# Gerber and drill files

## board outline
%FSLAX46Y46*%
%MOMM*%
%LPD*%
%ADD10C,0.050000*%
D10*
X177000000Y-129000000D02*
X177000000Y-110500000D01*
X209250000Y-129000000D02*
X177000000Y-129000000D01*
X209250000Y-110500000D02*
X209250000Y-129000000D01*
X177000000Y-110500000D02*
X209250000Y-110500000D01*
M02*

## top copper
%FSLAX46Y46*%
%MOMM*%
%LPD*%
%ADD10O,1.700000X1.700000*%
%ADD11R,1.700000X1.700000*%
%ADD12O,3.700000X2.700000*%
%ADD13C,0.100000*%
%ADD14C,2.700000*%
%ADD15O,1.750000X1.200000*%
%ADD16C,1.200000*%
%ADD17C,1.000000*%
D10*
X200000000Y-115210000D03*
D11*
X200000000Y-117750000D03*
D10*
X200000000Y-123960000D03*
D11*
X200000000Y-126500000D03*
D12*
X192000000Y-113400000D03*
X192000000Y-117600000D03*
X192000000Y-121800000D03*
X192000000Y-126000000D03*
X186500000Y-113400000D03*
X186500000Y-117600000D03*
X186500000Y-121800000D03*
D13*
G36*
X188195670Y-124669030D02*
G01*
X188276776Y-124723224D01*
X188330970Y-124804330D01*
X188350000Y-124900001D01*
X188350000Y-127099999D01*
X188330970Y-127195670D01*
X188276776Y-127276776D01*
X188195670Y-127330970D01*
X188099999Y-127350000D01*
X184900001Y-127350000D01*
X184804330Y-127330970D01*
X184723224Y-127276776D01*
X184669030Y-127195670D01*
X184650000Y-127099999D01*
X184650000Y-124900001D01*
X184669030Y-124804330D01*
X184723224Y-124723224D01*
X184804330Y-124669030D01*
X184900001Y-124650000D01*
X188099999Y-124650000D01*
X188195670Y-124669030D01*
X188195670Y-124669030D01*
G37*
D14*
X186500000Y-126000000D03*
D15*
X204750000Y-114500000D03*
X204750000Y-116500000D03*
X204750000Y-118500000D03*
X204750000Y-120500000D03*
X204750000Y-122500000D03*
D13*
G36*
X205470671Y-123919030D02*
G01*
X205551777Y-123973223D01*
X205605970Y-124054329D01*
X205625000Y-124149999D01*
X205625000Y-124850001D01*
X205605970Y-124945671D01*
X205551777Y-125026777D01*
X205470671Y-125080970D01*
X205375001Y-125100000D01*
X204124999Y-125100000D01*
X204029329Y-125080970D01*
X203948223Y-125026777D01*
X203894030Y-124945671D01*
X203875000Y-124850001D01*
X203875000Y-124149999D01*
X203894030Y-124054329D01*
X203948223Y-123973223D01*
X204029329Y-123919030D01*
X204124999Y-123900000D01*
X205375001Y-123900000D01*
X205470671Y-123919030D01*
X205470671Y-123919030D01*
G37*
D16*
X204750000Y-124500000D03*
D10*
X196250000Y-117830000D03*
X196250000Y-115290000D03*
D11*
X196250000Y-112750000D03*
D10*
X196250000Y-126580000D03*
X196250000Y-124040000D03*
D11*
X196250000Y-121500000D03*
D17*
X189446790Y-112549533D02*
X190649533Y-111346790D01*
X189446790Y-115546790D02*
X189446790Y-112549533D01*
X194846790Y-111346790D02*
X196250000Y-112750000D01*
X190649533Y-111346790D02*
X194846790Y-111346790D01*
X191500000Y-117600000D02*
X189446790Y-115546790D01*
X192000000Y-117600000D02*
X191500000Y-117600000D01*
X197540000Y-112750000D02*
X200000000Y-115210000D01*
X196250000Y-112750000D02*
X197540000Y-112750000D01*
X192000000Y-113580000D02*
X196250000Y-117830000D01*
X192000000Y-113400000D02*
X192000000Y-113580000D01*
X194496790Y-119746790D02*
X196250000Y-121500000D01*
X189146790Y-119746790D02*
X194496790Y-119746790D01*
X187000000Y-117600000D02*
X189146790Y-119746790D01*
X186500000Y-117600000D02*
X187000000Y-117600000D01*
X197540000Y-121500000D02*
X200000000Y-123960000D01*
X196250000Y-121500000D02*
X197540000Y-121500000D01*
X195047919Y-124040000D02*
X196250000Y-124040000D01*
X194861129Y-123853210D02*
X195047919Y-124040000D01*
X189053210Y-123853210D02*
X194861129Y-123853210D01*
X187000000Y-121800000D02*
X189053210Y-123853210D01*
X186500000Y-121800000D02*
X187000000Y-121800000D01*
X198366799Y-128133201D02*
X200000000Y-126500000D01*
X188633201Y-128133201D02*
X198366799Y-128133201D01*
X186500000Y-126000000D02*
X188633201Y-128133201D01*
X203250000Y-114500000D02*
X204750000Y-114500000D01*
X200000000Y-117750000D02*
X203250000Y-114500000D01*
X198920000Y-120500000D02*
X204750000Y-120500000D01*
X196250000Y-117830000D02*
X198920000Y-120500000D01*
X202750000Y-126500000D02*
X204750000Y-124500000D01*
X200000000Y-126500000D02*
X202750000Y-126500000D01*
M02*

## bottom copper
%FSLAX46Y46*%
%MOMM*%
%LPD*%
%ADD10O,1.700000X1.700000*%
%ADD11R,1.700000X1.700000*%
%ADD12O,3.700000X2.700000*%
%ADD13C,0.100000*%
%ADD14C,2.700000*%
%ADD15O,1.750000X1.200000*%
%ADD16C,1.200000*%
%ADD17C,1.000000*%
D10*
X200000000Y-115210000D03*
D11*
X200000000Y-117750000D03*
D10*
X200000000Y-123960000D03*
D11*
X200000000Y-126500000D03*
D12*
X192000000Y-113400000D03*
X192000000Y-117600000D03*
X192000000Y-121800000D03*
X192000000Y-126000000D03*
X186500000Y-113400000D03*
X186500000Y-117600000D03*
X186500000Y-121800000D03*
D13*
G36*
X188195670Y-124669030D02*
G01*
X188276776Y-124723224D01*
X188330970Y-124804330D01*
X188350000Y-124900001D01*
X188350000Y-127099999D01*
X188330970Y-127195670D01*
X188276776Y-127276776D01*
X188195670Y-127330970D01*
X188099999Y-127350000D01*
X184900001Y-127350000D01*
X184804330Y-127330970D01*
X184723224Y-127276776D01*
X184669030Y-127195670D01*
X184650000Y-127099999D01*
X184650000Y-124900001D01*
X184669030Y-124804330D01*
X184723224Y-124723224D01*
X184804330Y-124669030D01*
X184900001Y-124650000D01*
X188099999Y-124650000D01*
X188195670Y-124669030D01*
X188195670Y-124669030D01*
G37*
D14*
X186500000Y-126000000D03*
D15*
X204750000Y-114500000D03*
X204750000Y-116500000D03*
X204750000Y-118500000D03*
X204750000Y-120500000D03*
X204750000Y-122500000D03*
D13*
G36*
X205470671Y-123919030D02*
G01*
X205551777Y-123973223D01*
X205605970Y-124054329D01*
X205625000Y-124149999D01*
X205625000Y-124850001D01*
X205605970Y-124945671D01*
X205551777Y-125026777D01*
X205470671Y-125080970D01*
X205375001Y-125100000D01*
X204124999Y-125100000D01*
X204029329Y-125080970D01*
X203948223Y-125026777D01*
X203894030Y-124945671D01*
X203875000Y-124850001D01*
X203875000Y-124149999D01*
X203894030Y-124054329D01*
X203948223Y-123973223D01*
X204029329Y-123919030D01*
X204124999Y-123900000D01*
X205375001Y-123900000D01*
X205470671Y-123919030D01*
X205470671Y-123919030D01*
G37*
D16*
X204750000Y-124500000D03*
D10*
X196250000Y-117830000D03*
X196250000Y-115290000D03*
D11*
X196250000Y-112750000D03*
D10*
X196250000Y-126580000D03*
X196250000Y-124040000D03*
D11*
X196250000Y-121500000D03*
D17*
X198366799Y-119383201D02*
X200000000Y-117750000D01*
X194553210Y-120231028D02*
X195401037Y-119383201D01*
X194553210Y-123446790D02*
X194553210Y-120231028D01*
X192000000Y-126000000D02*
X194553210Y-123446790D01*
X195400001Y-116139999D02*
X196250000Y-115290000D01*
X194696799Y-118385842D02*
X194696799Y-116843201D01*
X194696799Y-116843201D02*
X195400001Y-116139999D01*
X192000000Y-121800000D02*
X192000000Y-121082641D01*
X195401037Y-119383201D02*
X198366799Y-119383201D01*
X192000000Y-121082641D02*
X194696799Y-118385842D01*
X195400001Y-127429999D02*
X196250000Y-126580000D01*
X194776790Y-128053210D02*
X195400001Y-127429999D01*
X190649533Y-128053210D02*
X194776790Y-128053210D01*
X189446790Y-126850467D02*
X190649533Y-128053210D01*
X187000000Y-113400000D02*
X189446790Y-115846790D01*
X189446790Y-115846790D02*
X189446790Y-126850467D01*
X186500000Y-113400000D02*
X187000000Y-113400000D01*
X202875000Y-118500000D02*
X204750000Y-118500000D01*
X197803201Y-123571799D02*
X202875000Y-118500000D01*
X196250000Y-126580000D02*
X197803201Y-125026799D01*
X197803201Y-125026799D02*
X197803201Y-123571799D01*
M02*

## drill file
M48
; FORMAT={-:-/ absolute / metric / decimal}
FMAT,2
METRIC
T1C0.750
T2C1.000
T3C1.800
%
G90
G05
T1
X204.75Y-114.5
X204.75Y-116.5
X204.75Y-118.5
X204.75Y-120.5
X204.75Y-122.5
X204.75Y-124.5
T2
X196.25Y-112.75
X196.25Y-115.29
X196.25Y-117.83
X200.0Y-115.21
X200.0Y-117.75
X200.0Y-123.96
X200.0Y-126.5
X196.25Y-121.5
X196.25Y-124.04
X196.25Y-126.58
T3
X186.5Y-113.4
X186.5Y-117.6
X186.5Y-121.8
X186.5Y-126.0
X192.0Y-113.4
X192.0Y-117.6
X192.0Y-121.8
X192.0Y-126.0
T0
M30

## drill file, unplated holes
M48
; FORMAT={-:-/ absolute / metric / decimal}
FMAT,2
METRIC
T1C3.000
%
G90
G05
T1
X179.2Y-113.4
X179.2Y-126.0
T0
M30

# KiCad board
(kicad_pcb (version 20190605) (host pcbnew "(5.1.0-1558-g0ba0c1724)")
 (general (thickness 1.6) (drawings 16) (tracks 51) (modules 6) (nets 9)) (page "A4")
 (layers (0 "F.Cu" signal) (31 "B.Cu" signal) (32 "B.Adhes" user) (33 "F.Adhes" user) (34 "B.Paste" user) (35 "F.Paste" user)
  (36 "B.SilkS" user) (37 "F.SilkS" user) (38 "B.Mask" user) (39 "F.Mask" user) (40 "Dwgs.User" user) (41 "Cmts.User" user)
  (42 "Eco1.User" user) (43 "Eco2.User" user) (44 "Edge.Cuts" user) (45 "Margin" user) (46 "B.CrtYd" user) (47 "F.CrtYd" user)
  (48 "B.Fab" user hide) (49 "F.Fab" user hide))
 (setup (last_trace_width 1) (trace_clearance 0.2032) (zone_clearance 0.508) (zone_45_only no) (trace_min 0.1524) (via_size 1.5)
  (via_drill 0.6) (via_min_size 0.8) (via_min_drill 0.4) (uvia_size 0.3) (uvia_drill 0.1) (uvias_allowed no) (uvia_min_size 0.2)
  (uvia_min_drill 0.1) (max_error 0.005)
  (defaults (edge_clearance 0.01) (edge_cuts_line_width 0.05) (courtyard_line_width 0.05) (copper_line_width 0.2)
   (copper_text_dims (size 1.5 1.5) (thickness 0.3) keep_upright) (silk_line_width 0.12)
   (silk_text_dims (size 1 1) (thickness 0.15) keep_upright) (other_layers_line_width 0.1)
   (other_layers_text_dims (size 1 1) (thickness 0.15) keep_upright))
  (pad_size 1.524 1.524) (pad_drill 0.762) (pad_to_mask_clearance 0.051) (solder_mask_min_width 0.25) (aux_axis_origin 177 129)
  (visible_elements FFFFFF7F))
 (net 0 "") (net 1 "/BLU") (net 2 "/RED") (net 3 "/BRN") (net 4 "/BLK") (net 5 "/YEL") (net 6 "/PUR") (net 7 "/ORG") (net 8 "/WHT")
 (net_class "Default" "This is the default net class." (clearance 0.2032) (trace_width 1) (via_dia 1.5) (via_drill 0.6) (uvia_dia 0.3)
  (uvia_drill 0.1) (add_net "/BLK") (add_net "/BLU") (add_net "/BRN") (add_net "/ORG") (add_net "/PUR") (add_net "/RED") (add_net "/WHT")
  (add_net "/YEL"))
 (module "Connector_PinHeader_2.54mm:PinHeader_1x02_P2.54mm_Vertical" (layer "F.Cu") (at 200 117.75 180)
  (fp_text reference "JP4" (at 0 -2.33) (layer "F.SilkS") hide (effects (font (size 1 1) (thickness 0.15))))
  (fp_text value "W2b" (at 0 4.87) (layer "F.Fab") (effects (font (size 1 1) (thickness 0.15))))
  (pad "2" thru_hole oval (at 0 2.54 180) (size 1.7 1.7) (drill 1) (layers *.Cu *.Mask) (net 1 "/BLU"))
  (pad "1" thru_hole rect (at 0 0 180) (size 1.7 1.7) (drill 1) (layers *.Cu *.Mask) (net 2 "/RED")))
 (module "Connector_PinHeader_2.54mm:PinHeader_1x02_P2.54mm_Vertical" (layer "F.Cu") (at 200 126.5 180)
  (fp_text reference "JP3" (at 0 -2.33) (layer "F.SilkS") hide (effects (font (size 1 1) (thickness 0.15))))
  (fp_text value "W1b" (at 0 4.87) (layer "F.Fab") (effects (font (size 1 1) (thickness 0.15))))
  (pad "2" thru_hole oval (at 0 2.54 180) (size 1.7 1.7) (drill 1) (layers *.Cu *.Mask) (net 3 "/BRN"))
  (pad "1" thru_hole rect (at 0 0 180) (size 1.7 1.7) (drill 1) (layers *.Cu *.Mask) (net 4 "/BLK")))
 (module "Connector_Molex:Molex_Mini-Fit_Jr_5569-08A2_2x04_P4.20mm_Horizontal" (layer "F.Cu") (at 186.5 126 90)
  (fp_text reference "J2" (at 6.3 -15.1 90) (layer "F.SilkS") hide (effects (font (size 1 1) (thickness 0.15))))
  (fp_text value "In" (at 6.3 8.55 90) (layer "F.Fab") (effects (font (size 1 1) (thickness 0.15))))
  (pad "" np_thru_hole circle (at 12.6 -7.3 90) (size 3 3) (drill 3) (layers *.Cu *.Mask))
  (pad "" np_thru_hole circle (at 0 -7.3 90) (size 3 3) (drill 3) (layers *.Cu *.Mask))
  (pad "8" thru_hole oval (at 12.6 5.5 90) (size 2.7 3.7) (drill 1.8) (layers *.Cu *.Mask) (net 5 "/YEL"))
  (pad "7" thru_hole oval (at 8.4 5.5 90) (size 2.7 3.7) (drill 1.8) (layers *.Cu *.Mask) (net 1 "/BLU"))
  (pad "6" thru_hole oval (at 4.2 5.5 90) (size 2.7 3.7) (drill 1.8) (layers *.Cu *.Mask) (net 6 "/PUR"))
  (pad "5" thru_hole oval (at 0 5.5 90) (size 2.7 3.7) (drill 1.8) (layers *.Cu *.Mask) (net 2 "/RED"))
  (pad "4" thru_hole oval (at 12.6 0 90) (size 2.7 3.7) (drill 1.8) (layers *.Cu *.Mask) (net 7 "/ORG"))
  (pad "3" thru_hole oval (at 8.4 0 90) (size 2.7 3.7) (drill 1.8) (layers *.Cu *.Mask) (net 3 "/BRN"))
  (pad "2" thru_hole oval (at 4.2 0 90) (size 2.7 3.7) (drill 1.8) (layers *.Cu *.Mask) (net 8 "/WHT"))
  (pad "1" thru_hole roundrect (at 0 0 90) (size 2.7 3.7) (drill 1.8) (layers *.Cu *.Mask) (roundrect_rratio 0.09259299999999999)
   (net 4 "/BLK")))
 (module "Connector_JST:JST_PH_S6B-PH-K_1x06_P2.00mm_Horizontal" (layer "F.Cu") (at 204.75 124.5 90)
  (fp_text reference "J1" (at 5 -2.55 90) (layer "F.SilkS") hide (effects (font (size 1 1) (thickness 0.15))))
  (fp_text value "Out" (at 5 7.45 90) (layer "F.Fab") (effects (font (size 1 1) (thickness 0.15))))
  (pad "6" thru_hole oval (at 10 0 90) (size 1.2 1.75) (drill 0.75) (layers *.Cu *.Mask) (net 2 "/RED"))
  (pad "5" thru_hole oval (at 8 0 90) (size 1.2 1.75) (drill 0.75) (layers *.Cu *.Mask))
  (pad "4" thru_hole oval (at 6 0 90) (size 1.2 1.75) (drill 0.75) (layers *.Cu *.Mask) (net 7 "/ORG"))
  (pad "3" thru_hole oval (at 4 0 90) (size 1.2 1.75) (drill 0.75) (layers *.Cu *.Mask) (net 5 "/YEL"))
  (pad "2" thru_hole oval (at 2 0 90) (size 1.2 1.75) (drill 0.75) (layers *.Cu *.Mask))
  (pad "1" thru_hole roundrect (at 0 0 90) (size 1.2 1.75) (drill 0.75) (layers *.Cu *.Mask) (roundrect_rratio 0.208333) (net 4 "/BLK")))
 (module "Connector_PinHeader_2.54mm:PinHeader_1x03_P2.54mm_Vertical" (layer "F.Cu") (at 196.25 112.75)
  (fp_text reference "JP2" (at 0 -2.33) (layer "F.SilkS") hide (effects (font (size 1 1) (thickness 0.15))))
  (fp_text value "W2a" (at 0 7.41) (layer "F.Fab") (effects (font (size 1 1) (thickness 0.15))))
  (pad "3" thru_hole oval (at 0 5.08) (size 1.7 1.7) (drill 1) (layers *.Cu *.Mask) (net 5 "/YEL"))
  (pad "2" thru_hole oval (at 0 2.54) (size 1.7 1.7) (drill 1) (layers *.Cu *.Mask) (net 6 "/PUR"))
  (pad "1" thru_hole rect (at 0 0) (size 1.7 1.7) (drill 1) (layers *.Cu *.Mask) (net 1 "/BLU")))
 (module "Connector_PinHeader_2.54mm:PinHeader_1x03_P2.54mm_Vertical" (layer "F.Cu") (at 196.25 121.5)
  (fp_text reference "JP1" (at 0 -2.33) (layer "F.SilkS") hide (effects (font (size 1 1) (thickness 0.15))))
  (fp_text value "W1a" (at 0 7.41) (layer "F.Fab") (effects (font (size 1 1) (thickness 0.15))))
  (pad "3" thru_hole oval (at 0 5.08) (size 1.7 1.7) (drill 1) (layers *.Cu *.Mask) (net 7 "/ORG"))
  (pad "2" thru_hole oval (at 0 2.54) (size 1.7 1.7) (drill 1) (layers *.Cu *.Mask) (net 8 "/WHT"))
  (pad "1" thru_hole rect (at 0 0) (size 1.7 1.7) (drill 1) (layers *.Cu *.Mask) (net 3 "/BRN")))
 (gr_line (start 177 129) (end 177 110.5) (layer "Edge.Cuts") (width 0.05))
 (gr_line (start 209.25 129) (end 177 129) (layer "Edge.Cuts") (width 0.05))
 (gr_line (start 209.25 110.5) (end 209.25 129) (layer "Edge.Cuts") (width 0.05))
 (gr_line (start 177 110.5) (end 209.25 110.5) (layer "Edge.Cuts") (width 0.05))
 (segment (start 189.44679 112.549533) (end 190.649533 111.34679) (width 1) (layer "F.Cu") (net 1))
 (segment (start 189.44679 115.54679) (end 189.44679 112.549533) (width 1) (layer "F.Cu") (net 1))
 (segment (start 194.84679 111.34679) (end 196.25 112.75) (width 1) (layer "F.Cu") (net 1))
 (segment (start 190.649533 111.34679) (end 194.84679 111.34679) (width 1) (layer "F.Cu") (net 1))
 (segment (start 191.5 117.6) (end 189.44679 115.54679) (width 1) (layer "F.Cu") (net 1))
 (segment (start 192 117.6) (end 191.5 117.6) (width 1) (layer "F.Cu") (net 1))
 (segment (start 197.54 112.75) (end 200 115.21) (width 1) (layer "F.Cu") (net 1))
 (segment (start 196.25 112.75) (end 197.54 112.75) (width 1) (layer "F.Cu") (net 1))
 (segment (start 192 113.58) (end 196.25 117.83) (width 1) (layer "F.Cu") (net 5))
 (segment (start 192 113.4) (end 192 113.58) (width 1) (layer "F.Cu") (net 5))
 (segment (start 194.49679 119.74679) (end 196.25 121.5) (width 1) (layer "F.Cu") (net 3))
 (segment (start 189.14679 119.74679) (end 194.49679 119.74679) (width 1) (layer "F.Cu") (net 3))
 (segment (start 187 117.6) (end 189.14679 119.74679) (width 1) (layer "F.Cu") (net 3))
 (segment (start 186.5 117.6) (end 187 117.6) (width 1) (layer "F.Cu") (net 3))
 (segment (start 197.54 121.5) (end 200 123.96) (width 1) (layer "F.Cu") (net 3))
 (segment (start 196.25 121.5) (end 197.54 121.5) (width 1) (layer "F.Cu") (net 3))
 (segment (start 195.047919 124.04) (end 196.25 124.04) (width 1) (layer "F.Cu") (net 8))
 (segment (start 194.861129 123.85321) (end 195.047919 124.04) (width 1) (layer "F.Cu") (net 8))
 (segment (start 189.05321 123.85321) (end 194.861129 123.85321) (width 1) (layer "F.Cu") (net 8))
 (segment (start 187 121.8) (end 189.05321 123.85321) (width 1) (layer "F.Cu") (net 8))
 (segment (start 186.5 121.8) (end 187 121.8) (width 1) (layer "F.Cu") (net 8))
 (segment (start 198.366799 128.133201) (end 200 126.5) (width 1) (layer "F.Cu") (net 4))
 (segment (start 188.633201 128.133201) (end 198.366799 128.133201) (width 1) (layer "F.Cu") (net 4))
 (segment (start 186.5 126) (end 188.633201 128.133201) (width 1) (layer "F.Cu") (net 4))
 (segment (start 203.25 114.5) (end 204.75 114.5) (width 1) (layer "F.Cu") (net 2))
 (segment (start 200 117.75) (end 203.25 114.5) (width 1) (layer "F.Cu") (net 2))
 (segment (start 198.92 120.5) (end 204.75 120.5) (width 1) (layer "F.Cu") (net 5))
 (segment (start 196.25 117.83) (end 198.92 120.5) (width 1) (layer "F.Cu") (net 5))
 (segment (start 202.75 126.5) (end 204.75 124.5) (width 1) (layer "F.Cu") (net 4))
 (segment (start 200 126.5) (end 202.75 126.5) (width 1) (layer "F.Cu") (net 4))
 (segment (start 198.366799 119.383201) (end 200 117.75) (width 1) (layer "B.Cu") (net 2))
 (segment (start 194.55321 120.231028) (end 195.401037 119.383201) (width 1) (layer "B.Cu") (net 2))
 (segment (start 194.55321 123.44679) (end 194.55321 120.231028) (width 1) (layer "B.Cu") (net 2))
 (segment (start 192 126) (end 194.55321 123.44679) (width 1) (layer "B.Cu") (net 2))
 (segment (start 195.400001 116.139999) (end 196.25 115.29) (width 1) (layer "B.Cu") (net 6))
 (segment (start 194.696799 118.385842) (end 194.696799 116.843201) (width 1) (layer "B.Cu") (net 6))
 (segment (start 194.696799 116.843201) (end 195.400001 116.139999) (width 1) (layer "B.Cu") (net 6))
 (segment (start 192 121.8) (end 192 121.082641) (width 1) (layer "B.Cu") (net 6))
 (segment (start 195.401037 119.383201) (end 198.366799 119.383201) (width 1) (layer "B.Cu") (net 2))
 (segment (start 192 121.082641) (end 194.696799 118.385842) (width 1) (layer "B.Cu") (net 6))
 (segment (start 195.400001 127.429999) (end 196.25 126.58) (width 1) (layer "B.Cu") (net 7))
 (segment (start 194.77679 128.05321) (end 195.400001 127.429999) (width 1) (layer "B.Cu") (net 7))
 (segment (start 190.649533 128.05321) (end 194.77679 128.05321) (width 1) (layer "B.Cu") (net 7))
 (segment (start 189.44679 126.850467) (end 190.649533 128.05321) (width 1) (layer "B.Cu") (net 7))
 (segment (start 187 113.4) (end 189.44679 115.84679) (width 1) (layer "B.Cu") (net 7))
 (segment (start 189.44679 115.84679) (end 189.44679 126.850467) (width 1) (layer "B.Cu") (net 7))
 (segment (start 186.5 113.4) (end 187 113.4) (width 1) (layer "B.Cu") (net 7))
 (segment (start 202.875 118.5) (end 204.75 118.5) (width 1) (layer "B.Cu") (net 7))
 (segment (start 197.803201 123.571799) (end 202.875 118.5) (width 1) (layer "B.Cu") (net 7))
 (segment (start 196.25 126.58) (end 197.803201 125.026799) (width 1) (layer "B.Cu") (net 7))
 (segment (start 197.803201 125.026799) (end 197.803201 123.571799) (width 1) (layer "B.Cu") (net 7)))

